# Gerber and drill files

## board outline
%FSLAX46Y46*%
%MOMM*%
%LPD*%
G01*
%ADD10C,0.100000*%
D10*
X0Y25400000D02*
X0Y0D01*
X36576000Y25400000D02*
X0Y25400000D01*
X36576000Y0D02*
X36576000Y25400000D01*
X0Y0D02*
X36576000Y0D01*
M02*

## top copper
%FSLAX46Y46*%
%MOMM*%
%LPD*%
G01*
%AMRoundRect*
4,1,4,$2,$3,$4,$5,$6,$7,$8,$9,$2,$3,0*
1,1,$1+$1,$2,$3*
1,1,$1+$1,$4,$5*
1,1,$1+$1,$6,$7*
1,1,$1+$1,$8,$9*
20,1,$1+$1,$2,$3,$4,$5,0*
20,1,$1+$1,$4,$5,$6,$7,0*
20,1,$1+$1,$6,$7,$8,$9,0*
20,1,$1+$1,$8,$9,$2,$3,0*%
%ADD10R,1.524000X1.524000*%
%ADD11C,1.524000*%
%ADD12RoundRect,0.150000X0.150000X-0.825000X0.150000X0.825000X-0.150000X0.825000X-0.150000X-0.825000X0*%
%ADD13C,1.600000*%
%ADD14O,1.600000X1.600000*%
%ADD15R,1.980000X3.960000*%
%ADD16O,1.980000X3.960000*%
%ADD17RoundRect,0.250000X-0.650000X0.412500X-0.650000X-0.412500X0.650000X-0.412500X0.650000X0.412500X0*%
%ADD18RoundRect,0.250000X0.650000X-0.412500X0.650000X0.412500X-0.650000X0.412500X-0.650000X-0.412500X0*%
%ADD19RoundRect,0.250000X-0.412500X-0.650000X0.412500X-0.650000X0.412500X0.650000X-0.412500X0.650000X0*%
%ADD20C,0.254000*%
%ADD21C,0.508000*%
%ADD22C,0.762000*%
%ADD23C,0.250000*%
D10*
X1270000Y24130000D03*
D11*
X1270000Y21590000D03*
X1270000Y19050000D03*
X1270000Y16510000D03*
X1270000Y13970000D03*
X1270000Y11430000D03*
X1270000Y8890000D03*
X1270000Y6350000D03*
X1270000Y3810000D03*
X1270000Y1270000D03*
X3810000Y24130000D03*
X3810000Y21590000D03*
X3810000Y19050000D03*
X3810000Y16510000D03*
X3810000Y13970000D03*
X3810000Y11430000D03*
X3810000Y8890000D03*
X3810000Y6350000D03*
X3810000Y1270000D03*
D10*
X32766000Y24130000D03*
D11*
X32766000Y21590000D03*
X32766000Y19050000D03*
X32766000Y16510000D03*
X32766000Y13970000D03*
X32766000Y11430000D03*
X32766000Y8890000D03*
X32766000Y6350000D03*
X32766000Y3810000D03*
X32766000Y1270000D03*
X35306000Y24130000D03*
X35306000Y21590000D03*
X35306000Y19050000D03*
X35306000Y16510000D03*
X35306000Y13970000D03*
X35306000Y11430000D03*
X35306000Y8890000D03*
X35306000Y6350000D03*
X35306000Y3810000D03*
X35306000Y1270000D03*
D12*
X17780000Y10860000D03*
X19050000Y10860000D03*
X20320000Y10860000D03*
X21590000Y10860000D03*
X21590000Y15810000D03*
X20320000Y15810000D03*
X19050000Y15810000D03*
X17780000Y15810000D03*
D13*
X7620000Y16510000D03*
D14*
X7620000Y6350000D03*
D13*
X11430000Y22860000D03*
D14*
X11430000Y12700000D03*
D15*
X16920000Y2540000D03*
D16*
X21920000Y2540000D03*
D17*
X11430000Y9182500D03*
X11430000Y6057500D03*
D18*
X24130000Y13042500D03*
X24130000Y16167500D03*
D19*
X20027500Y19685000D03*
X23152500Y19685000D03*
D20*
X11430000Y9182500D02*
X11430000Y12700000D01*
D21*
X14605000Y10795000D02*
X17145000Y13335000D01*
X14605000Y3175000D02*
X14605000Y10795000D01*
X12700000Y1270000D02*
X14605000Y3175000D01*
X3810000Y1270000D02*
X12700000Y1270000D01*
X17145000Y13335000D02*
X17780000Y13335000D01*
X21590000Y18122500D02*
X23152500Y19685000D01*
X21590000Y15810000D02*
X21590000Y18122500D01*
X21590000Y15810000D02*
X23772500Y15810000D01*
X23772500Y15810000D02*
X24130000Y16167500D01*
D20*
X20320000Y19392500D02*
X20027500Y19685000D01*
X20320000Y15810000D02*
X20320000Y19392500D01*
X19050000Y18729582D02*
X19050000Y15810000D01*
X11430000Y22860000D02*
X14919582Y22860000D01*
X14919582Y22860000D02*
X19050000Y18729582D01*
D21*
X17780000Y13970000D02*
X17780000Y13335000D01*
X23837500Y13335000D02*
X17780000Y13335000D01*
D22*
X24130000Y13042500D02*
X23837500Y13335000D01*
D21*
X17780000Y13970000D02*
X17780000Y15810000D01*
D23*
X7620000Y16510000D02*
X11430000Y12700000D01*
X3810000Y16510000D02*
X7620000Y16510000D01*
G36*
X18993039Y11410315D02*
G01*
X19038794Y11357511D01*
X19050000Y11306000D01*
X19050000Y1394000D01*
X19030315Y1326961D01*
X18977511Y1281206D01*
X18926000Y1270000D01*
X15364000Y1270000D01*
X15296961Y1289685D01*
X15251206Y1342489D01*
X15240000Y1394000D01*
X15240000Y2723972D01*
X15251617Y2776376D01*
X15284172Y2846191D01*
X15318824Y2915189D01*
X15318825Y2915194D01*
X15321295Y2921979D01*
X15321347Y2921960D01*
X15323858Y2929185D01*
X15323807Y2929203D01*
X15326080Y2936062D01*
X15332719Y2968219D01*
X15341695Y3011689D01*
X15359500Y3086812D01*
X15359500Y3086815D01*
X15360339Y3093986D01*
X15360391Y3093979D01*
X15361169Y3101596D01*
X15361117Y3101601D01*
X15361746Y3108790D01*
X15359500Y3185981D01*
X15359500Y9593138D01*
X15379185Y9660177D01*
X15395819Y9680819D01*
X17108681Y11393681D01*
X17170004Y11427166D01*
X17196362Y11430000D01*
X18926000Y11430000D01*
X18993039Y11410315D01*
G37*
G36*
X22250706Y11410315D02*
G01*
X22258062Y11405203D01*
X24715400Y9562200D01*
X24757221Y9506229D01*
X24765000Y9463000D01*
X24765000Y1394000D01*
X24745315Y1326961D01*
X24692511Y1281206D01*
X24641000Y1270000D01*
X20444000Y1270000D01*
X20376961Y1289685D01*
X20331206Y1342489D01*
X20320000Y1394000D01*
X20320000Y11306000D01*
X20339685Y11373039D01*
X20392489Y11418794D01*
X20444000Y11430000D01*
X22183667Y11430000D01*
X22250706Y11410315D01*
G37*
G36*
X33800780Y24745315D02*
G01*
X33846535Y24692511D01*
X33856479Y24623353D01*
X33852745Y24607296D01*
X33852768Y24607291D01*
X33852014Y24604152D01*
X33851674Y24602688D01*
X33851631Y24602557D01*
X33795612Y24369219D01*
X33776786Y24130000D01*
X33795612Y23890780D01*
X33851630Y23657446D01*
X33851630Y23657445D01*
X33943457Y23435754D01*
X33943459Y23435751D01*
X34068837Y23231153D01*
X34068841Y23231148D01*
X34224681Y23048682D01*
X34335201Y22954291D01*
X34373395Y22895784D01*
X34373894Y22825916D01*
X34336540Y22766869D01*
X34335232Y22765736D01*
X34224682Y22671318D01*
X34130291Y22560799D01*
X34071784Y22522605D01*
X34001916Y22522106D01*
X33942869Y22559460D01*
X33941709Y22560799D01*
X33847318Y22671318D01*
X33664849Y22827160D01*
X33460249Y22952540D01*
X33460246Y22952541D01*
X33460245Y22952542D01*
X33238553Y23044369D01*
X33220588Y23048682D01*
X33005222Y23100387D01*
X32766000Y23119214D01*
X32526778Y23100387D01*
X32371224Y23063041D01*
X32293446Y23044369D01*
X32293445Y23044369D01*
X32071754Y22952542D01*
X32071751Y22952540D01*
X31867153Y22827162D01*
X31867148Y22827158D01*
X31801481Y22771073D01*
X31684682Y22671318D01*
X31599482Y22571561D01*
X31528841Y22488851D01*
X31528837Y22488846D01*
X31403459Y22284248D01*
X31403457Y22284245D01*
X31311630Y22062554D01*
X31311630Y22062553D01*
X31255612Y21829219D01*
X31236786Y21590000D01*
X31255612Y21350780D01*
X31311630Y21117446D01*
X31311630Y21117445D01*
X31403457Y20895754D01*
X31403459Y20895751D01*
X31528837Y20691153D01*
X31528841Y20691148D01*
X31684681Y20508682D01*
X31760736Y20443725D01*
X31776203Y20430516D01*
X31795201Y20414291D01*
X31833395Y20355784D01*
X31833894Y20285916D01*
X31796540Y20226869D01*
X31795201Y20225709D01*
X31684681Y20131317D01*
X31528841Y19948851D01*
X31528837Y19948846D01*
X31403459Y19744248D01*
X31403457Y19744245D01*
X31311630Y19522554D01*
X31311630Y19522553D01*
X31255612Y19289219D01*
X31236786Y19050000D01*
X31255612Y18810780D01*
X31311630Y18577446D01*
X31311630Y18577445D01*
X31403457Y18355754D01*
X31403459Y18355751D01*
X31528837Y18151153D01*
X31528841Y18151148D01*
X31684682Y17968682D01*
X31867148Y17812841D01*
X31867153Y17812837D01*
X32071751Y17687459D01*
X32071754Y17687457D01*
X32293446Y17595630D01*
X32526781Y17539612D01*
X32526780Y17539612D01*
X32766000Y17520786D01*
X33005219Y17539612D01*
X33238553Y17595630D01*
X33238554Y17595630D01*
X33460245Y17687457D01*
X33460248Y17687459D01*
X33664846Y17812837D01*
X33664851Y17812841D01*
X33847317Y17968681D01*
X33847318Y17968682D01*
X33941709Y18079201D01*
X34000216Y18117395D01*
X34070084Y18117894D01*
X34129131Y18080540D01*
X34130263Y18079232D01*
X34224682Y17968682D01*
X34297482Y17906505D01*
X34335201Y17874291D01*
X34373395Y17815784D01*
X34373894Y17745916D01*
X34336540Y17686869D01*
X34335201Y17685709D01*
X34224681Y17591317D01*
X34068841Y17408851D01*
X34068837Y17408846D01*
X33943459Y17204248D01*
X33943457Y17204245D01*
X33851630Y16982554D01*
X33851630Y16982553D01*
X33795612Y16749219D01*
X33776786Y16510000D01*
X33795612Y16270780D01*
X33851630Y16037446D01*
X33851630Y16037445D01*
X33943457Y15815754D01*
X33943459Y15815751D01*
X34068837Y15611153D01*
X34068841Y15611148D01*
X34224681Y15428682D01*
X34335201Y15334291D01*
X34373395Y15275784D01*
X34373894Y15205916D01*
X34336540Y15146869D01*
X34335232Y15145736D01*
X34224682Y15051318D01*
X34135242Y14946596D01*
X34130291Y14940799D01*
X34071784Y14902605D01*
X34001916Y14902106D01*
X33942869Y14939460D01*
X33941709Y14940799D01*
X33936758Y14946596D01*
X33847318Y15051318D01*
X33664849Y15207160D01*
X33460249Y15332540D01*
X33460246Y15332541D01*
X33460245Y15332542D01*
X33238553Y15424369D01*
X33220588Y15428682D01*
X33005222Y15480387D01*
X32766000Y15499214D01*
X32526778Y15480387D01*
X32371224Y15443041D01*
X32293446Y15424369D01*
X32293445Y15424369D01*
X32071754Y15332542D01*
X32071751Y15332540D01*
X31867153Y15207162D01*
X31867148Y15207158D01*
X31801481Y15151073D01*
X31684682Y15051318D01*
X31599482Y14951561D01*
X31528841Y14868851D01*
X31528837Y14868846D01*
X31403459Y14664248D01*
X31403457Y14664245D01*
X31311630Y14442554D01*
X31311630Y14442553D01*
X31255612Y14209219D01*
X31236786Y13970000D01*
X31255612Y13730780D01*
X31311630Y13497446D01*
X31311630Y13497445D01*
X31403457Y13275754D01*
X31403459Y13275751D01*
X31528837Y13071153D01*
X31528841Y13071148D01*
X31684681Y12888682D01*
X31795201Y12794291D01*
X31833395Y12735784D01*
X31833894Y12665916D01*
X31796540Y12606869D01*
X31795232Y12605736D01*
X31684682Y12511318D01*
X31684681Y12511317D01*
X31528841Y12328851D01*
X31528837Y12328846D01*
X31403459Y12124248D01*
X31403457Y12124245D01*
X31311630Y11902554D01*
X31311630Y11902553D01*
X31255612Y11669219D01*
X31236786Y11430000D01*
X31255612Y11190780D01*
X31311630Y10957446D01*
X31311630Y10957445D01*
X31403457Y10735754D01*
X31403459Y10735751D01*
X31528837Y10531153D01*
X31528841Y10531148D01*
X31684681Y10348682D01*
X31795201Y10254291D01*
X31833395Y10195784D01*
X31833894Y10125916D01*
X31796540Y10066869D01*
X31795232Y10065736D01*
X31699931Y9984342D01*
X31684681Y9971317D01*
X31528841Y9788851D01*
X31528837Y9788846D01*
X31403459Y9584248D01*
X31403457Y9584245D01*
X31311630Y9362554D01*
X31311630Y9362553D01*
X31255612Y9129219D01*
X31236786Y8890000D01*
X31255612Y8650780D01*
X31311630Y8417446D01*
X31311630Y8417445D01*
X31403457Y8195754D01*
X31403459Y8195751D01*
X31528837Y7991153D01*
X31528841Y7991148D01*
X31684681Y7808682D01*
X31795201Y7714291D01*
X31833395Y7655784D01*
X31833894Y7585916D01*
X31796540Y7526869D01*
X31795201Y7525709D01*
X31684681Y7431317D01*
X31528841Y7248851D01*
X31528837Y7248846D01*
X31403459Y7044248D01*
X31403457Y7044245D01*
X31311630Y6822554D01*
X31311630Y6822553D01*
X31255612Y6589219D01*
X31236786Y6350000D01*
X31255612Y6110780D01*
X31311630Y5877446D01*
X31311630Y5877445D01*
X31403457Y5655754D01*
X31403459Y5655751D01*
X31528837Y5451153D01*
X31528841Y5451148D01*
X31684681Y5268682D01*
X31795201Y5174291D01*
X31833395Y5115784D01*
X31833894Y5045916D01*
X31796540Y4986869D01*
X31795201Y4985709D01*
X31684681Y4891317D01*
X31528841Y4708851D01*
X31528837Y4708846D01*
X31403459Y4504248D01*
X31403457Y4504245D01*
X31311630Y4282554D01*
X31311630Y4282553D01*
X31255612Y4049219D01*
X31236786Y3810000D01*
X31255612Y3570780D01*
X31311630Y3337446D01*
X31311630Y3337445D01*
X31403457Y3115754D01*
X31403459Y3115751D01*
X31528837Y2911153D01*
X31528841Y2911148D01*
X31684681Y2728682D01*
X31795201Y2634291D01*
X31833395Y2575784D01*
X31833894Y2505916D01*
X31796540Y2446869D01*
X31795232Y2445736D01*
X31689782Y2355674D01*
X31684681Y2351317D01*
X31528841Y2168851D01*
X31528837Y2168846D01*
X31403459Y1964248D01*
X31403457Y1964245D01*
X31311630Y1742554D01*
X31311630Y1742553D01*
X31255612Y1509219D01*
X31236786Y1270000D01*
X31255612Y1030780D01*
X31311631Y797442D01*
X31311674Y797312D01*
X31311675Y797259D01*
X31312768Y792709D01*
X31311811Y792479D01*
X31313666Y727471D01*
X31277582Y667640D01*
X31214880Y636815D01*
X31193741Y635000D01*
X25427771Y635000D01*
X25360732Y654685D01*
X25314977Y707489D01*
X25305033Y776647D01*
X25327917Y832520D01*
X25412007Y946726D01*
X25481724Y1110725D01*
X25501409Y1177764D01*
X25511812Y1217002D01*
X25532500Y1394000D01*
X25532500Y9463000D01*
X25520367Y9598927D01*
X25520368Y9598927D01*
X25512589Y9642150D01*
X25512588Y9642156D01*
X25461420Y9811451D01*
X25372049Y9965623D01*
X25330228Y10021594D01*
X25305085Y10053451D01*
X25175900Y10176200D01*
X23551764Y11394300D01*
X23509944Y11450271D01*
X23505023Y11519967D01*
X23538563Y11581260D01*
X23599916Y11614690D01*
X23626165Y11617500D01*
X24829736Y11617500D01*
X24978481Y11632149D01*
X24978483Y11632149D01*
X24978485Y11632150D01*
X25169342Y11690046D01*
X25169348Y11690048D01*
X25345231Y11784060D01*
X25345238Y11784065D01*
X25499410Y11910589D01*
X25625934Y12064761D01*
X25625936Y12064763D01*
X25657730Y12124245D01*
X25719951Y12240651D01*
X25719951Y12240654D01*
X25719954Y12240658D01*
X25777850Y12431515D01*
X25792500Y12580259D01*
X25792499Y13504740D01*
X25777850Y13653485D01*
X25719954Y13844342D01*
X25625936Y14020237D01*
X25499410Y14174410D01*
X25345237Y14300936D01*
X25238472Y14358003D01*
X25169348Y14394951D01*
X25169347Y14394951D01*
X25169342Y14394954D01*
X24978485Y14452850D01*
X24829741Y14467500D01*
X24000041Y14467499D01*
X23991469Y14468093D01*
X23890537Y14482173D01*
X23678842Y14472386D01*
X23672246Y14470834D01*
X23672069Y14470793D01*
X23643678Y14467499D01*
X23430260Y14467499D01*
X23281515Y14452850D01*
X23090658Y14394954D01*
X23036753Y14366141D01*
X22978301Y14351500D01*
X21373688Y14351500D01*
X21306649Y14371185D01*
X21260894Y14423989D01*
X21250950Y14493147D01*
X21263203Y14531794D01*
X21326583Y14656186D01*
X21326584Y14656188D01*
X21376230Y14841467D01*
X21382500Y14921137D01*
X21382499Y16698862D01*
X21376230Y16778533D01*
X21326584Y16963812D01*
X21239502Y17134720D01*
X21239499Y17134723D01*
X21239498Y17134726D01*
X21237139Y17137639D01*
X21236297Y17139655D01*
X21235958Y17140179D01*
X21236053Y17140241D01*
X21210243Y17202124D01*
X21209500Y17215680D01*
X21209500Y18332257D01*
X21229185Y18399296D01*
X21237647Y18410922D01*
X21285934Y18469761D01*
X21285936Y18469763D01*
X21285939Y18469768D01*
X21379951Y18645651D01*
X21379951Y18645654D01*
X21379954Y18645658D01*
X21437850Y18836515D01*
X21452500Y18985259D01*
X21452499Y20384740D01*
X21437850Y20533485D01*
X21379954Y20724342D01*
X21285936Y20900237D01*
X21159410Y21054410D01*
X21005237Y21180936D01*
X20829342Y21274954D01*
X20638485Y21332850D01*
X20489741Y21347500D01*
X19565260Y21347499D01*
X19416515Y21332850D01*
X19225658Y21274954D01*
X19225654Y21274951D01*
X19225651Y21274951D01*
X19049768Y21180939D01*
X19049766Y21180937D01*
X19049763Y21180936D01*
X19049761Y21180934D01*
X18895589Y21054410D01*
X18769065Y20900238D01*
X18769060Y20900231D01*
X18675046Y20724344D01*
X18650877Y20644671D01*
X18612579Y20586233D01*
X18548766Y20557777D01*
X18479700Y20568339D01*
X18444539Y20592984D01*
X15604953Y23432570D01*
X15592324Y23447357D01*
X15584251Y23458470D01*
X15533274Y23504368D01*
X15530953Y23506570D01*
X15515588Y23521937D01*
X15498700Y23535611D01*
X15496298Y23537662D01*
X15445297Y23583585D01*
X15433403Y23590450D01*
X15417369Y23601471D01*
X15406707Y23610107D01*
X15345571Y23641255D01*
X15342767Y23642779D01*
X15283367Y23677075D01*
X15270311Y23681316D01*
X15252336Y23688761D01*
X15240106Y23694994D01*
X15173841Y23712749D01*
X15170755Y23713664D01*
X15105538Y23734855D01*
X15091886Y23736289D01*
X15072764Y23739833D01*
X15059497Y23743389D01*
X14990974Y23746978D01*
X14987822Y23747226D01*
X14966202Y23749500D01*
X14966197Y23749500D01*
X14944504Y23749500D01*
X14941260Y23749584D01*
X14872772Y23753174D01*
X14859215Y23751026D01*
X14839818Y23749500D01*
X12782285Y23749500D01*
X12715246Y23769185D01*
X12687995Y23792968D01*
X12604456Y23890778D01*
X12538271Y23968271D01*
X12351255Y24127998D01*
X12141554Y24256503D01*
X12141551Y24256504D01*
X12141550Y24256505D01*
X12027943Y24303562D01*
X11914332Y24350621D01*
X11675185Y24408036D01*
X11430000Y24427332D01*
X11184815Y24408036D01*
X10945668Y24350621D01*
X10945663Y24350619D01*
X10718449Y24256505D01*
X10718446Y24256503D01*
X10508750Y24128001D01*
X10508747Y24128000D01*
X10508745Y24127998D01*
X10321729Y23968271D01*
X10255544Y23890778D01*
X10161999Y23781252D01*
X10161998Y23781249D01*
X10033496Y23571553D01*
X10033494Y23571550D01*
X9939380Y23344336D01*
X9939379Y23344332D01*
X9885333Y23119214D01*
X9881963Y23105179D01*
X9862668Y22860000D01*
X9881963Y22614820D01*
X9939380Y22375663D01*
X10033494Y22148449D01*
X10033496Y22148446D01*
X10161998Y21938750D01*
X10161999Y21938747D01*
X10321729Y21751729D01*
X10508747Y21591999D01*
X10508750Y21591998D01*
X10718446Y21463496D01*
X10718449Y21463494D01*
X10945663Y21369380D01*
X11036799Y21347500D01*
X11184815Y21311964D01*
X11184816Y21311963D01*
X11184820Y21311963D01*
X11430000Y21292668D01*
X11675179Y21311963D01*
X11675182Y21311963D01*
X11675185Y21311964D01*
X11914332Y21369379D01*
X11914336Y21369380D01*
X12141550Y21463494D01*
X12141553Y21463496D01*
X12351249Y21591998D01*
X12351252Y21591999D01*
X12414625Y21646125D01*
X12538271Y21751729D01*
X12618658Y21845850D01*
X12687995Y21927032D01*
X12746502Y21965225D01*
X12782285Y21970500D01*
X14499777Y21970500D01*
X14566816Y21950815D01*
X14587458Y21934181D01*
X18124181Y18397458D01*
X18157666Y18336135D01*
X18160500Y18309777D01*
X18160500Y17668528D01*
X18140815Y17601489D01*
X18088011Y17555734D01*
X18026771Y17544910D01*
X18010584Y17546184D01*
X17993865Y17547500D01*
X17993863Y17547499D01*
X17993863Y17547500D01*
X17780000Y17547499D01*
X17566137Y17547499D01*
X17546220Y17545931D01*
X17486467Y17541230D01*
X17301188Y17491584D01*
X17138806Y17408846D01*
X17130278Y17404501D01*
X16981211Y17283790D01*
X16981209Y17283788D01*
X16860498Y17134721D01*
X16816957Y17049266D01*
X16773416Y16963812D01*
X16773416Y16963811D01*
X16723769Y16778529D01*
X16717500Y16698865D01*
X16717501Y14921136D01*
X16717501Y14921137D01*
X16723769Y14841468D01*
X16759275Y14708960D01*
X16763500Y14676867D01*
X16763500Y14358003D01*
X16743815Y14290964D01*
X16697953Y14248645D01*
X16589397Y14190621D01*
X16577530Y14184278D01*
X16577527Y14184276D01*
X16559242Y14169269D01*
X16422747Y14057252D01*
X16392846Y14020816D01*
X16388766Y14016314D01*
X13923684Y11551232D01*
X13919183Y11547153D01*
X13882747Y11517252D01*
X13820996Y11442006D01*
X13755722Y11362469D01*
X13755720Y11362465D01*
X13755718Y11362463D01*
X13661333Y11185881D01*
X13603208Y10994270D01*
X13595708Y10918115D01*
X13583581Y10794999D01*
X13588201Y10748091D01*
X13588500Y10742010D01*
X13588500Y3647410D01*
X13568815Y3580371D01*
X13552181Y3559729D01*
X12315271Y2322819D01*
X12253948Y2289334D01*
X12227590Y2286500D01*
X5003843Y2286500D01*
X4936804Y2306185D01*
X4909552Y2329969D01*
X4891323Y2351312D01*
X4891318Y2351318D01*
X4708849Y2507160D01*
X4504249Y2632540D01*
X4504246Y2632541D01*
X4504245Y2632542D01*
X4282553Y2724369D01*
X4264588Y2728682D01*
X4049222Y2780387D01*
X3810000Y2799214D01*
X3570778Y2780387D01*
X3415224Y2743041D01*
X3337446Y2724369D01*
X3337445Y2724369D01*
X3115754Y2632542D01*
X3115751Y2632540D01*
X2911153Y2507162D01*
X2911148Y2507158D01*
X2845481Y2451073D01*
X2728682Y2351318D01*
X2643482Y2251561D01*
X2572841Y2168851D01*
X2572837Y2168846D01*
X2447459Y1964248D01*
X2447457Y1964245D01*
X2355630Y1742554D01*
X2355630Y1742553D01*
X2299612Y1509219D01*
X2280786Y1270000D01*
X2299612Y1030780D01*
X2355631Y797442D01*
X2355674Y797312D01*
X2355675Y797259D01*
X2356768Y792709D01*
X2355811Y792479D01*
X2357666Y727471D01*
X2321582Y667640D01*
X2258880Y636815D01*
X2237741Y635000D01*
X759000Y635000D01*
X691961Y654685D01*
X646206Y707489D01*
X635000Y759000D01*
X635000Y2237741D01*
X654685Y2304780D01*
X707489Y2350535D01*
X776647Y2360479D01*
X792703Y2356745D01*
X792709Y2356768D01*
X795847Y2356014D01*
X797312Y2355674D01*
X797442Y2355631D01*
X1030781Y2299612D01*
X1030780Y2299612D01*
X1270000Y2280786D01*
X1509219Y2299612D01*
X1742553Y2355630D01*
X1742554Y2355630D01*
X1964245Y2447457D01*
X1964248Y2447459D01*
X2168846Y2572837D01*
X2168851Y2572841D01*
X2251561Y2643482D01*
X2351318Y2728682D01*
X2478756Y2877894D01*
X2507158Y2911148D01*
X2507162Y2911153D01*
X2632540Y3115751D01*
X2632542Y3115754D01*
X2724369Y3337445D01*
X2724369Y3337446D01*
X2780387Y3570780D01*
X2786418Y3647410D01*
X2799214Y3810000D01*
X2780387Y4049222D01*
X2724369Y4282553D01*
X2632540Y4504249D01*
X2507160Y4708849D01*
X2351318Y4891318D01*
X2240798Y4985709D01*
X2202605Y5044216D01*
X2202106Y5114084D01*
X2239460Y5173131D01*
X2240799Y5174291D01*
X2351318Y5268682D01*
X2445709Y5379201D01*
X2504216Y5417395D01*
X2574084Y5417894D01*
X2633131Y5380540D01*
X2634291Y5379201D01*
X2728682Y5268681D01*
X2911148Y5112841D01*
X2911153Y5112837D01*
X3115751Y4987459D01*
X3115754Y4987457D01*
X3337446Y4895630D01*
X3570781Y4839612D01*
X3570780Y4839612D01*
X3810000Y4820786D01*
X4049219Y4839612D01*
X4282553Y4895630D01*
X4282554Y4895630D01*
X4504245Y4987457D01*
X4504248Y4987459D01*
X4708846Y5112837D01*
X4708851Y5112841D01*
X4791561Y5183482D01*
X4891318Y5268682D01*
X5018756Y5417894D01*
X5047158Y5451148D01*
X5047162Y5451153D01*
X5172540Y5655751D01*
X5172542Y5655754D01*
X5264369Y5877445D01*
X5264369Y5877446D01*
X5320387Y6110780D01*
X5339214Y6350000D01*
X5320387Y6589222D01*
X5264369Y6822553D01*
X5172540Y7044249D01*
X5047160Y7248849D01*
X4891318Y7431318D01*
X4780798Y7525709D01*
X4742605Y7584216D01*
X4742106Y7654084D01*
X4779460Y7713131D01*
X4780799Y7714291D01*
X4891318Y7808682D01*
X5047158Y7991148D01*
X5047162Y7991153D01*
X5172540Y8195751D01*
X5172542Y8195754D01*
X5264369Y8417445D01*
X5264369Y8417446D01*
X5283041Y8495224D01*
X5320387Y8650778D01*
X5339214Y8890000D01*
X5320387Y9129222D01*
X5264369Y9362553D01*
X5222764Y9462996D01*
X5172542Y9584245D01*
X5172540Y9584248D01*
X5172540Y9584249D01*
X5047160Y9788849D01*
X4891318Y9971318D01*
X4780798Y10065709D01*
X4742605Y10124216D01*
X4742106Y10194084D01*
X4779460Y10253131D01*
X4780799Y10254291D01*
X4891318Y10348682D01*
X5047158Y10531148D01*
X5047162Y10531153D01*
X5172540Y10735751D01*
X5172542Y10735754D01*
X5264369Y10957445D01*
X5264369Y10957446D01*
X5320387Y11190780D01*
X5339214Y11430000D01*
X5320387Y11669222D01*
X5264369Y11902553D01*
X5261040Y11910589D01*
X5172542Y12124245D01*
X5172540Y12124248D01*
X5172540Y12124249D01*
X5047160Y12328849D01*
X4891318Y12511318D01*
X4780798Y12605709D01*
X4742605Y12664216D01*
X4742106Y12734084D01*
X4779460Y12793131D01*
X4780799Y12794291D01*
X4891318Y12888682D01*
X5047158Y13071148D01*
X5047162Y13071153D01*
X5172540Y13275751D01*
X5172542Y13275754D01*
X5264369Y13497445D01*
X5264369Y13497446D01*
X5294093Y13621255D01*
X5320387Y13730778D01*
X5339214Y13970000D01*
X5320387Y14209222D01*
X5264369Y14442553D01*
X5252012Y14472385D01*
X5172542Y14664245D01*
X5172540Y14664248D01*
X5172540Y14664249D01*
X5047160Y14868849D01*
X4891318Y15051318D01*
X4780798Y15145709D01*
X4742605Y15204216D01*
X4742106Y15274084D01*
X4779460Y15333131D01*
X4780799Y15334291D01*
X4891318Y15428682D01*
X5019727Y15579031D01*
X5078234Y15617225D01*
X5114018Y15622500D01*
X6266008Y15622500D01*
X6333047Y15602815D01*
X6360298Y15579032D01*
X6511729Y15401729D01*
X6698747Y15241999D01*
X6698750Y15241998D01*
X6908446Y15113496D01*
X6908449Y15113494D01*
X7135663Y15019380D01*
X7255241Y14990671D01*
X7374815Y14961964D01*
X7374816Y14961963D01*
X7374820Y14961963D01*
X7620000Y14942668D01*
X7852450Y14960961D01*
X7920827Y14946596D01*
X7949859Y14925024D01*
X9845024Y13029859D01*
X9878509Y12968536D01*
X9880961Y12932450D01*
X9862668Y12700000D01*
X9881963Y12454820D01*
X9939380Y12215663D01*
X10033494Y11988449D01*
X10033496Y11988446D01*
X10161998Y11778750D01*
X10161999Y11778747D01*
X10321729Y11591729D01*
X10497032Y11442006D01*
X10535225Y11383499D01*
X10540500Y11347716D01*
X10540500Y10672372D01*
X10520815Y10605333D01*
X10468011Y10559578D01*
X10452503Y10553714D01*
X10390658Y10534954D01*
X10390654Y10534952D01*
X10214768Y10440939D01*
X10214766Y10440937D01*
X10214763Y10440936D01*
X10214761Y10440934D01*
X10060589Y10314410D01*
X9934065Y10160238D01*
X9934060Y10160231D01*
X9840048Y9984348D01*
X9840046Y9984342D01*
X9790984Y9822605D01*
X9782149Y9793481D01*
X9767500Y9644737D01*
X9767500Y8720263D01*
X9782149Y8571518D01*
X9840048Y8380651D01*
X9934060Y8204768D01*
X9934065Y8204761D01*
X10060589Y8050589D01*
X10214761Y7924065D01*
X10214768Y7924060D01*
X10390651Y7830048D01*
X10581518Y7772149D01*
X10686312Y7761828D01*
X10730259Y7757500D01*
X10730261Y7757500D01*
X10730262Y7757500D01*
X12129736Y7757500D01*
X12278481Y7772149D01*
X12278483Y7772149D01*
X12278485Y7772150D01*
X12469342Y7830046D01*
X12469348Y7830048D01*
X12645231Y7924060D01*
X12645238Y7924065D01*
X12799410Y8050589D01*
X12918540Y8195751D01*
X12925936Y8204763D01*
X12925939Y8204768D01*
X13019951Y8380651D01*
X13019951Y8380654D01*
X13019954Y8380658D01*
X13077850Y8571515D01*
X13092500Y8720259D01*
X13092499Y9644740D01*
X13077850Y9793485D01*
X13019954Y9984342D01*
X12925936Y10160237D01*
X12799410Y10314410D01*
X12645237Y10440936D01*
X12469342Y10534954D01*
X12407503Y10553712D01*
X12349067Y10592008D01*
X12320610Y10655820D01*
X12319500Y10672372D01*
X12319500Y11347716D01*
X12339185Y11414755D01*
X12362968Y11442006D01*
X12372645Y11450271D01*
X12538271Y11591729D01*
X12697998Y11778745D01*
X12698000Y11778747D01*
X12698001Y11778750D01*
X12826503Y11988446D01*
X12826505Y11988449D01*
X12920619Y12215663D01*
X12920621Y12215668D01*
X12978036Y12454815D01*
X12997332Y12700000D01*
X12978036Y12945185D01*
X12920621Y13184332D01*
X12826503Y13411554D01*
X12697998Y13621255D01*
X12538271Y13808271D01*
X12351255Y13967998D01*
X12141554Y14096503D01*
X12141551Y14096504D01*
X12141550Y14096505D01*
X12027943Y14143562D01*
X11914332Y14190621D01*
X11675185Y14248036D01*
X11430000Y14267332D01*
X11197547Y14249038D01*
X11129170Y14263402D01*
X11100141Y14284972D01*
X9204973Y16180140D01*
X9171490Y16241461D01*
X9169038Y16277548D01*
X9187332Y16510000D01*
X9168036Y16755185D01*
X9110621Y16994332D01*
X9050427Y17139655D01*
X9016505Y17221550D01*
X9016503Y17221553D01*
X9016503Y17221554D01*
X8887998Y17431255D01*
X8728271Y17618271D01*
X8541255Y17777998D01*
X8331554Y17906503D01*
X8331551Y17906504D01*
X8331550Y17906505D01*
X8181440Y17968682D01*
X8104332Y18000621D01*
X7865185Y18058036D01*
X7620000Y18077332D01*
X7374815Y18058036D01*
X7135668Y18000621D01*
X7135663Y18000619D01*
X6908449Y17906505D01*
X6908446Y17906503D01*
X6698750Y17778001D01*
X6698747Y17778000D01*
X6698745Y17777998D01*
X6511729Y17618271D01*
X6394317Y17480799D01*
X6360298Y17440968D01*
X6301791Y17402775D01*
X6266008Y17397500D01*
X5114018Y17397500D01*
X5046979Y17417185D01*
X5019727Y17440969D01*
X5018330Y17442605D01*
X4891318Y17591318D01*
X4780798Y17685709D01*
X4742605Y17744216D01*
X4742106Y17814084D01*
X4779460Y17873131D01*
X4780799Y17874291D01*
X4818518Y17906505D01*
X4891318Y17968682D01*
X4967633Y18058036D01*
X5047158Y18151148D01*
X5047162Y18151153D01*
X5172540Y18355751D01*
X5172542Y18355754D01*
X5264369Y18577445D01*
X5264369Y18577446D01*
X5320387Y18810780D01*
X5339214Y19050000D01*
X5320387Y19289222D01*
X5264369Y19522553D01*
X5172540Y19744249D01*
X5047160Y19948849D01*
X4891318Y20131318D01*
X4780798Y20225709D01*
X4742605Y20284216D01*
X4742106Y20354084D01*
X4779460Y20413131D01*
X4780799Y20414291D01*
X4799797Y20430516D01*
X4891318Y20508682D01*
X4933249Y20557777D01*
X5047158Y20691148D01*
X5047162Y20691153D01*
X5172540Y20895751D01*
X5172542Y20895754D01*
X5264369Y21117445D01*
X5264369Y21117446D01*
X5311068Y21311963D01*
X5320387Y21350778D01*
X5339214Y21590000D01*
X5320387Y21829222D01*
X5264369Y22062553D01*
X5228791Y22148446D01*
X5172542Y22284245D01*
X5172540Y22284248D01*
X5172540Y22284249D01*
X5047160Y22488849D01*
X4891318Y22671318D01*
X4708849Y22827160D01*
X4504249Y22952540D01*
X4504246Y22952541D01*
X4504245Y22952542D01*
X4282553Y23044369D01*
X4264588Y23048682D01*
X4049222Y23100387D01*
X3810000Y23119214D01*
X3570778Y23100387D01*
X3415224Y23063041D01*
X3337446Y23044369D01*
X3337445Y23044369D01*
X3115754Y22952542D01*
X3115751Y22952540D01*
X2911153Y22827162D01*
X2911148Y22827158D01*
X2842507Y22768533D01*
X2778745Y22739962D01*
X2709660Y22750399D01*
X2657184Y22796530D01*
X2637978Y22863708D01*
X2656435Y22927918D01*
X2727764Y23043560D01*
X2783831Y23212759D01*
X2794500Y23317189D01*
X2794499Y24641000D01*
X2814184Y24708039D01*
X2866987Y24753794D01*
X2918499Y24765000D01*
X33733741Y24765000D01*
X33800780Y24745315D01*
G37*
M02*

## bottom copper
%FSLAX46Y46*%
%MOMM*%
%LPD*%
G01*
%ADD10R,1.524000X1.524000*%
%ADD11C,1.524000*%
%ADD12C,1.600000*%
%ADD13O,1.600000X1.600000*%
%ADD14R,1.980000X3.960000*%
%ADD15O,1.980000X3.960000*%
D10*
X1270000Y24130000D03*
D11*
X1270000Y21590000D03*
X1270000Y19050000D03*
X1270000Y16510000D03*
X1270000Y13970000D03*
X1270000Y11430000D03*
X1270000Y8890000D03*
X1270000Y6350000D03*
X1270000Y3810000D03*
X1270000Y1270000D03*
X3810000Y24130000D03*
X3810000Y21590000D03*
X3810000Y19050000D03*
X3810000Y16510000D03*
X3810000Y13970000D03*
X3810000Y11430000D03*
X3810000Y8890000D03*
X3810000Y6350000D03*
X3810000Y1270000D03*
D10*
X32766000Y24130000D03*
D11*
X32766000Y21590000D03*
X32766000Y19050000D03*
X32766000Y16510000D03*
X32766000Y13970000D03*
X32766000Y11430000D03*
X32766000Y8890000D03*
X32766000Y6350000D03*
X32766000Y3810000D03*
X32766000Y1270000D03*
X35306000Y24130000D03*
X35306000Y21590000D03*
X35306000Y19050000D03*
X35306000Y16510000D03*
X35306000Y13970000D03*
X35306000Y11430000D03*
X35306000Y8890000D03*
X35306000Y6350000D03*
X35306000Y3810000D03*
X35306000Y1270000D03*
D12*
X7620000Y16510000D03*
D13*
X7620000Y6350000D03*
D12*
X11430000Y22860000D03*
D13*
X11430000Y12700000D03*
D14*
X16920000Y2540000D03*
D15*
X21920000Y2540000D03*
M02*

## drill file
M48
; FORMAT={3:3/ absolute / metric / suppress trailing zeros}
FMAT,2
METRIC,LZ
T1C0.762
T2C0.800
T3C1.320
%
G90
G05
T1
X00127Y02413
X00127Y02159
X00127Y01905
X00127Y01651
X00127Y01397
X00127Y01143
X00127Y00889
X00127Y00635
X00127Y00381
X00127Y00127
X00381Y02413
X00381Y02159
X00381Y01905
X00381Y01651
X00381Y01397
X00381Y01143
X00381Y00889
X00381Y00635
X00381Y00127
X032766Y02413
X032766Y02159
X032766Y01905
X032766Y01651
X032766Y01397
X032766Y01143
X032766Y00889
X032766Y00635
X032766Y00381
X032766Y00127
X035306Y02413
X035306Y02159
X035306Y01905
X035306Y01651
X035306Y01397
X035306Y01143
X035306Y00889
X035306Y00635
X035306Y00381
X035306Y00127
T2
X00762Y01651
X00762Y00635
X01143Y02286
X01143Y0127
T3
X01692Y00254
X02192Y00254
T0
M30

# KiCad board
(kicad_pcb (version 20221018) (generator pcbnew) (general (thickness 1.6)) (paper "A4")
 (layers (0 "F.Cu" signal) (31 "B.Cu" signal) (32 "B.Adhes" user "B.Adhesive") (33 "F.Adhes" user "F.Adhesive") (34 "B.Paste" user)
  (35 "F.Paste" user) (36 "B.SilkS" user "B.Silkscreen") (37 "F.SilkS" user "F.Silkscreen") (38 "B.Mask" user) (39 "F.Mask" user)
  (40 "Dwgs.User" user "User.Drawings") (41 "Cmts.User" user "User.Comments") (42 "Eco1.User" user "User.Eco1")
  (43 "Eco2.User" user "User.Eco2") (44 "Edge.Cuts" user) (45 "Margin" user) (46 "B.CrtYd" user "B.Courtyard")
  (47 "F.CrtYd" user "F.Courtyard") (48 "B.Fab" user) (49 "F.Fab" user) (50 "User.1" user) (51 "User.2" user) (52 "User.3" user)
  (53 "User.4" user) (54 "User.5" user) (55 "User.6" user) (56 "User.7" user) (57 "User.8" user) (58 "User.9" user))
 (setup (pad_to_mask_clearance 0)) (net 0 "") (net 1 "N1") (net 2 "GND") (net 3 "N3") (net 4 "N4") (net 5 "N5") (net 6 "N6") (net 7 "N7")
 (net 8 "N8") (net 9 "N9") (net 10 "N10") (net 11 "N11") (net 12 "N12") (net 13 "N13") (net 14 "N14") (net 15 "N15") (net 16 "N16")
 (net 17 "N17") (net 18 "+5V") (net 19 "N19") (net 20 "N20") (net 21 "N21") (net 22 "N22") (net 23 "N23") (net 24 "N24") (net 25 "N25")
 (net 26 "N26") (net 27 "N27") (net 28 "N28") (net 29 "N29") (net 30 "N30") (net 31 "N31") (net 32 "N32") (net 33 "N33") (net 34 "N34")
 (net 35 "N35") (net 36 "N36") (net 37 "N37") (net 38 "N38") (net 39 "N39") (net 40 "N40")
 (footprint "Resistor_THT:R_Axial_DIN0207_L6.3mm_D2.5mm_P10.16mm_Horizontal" (layer "F.Cu") (at 7.62 -16.51 -90)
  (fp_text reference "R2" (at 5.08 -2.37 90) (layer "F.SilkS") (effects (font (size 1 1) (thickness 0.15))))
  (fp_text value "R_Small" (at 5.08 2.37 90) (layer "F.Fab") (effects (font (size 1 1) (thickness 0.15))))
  (pad "1" thru_hole circle (at 0 0 270) (size 1.6 1.6) (drill 0.8) (layers "*.Cu" "*.Mask") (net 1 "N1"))
  (pad "2" thru_hole oval (at 10.16 0 270) (size 1.6 1.6) (drill 0.8) (layers "*.Cu" "*.Mask") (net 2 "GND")))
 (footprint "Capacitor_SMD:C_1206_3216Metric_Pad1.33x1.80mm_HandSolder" (layer "F.Cu") (at 11.43 -7.62 -90)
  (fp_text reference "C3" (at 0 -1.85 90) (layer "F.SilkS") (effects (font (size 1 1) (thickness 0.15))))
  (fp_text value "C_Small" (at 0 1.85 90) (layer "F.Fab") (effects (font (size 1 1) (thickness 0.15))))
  (pad "1" smd roundrect (at -1.5625 0 270) (size 1.325 1.8) (layers "F.Cu" "F.Paste" "F.Mask") (roundrect_rratio 0.1886792453) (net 1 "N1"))
  (pad "2" smd roundrect (at 1.5625 0 270) (size 1.325 1.8) (layers "F.Cu" "F.Paste" "F.Mask") (roundrect_rratio 0.1886792453) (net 2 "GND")))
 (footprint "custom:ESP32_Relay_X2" (layer "F.Cu") (at 35.306 -13.97)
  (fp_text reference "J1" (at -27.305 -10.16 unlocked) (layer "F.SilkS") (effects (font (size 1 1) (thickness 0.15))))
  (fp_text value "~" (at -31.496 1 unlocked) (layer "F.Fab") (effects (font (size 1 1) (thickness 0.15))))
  (pad "1" thru_hole rect (at -34.036 -10.16) (size 1.524 1.524) (drill 0.762) (layers "*.Cu" "*.Mask") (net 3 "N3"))
  (pad "2" thru_hole circle (at -34.036 -7.62) (size 1.524 1.524) (drill 0.762) (layers "*.Cu" "*.Mask") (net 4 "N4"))
  (pad "3" thru_hole circle (at -34.036 -5.08) (size 1.524 1.524) (drill 0.762) (layers "*.Cu" "*.Mask") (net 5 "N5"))
  (pad "4" thru_hole circle (at -34.036 -2.54) (size 1.524 1.524) (drill 0.762) (layers "*.Cu" "*.Mask") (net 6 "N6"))
  (pad "5" thru_hole circle (at -34.036 0) (size 1.524 1.524) (drill 0.762) (layers "*.Cu" "*.Mask") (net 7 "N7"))
  (pad "6" thru_hole circle (at -34.036 2.54) (size 1.524 1.524) (drill 0.762) (layers "*.Cu" "*.Mask") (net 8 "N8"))
  (pad "7" thru_hole circle (at -34.036 5.08) (size 1.524 1.524) (drill 0.762) (layers "*.Cu" "*.Mask") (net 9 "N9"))
  (pad "8" thru_hole circle (at -34.036 7.62) (size 1.524 1.524) (drill 0.762) (layers "*.Cu" "*.Mask") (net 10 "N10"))
  (pad "9" thru_hole circle (at -34.036 10.16) (size 1.524 1.524) (drill 0.762) (layers "*.Cu" "*.Mask") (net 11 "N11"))
  (pad "10" thru_hole circle (at -34.036 12.7) (size 1.524 1.524) (drill 0.762) (layers "*.Cu" "*.Mask") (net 2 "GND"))
  (pad "11" thru_hole circle (at -31.496 -10.16) (size 1.524 1.524) (drill 0.762) (layers "*.Cu" "*.Mask") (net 2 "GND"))
  (pad "12" thru_hole circle (at -31.496 -7.62) (size 1.524 1.524) (drill 0.762) (layers "*.Cu" "*.Mask") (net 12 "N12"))
  (pad "13" thru_hole circle (at -31.496 -5.08) (size 1.524 1.524) (drill 0.762) (layers "*.Cu" "*.Mask") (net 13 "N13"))
  (pad "14" thru_hole circle (at -31.496 -2.54) (size 1.524 1.524) (drill 0.762) (layers "*.Cu" "*.Mask") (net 1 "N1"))
  (pad "15" thru_hole circle (at -31.496 0) (size 1.524 1.524) (drill 0.762) (layers "*.Cu" "*.Mask") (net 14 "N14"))
  (pad "16" thru_hole circle (at -31.496 2.54) (size 1.524 1.524) (drill 0.762) (layers "*.Cu" "*.Mask") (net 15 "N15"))
  (pad "17" thru_hole circle (at -31.496 5.08) (size 1.524 1.524) (drill 0.762) (layers "*.Cu" "*.Mask") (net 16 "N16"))
  (pad "18" thru_hole circle (at -31.496 7.62) (size 1.524 1.524) (drill 0.762) (layers "*.Cu" "*.Mask") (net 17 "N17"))
  (pad "20" thru_hole circle (at -31.496 12.7) (size 1.524 1.524) (drill 0.762) (layers "*.Cu" "*.Mask") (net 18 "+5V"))
  (pad "21" thru_hole rect (at -2.54 -10.16) (size 1.524 1.524) (drill 0.762) (layers "*.Cu" "*.Mask") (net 2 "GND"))
  (pad "22" thru_hole circle (at -2.54 -7.62) (size 1.524 1.524) (drill 0.762) (layers "*.Cu" "*.Mask") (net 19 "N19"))
  (pad "23" thru_hole circle (at -2.54 -5.08) (size 1.524 1.524) (drill 0.762) (layers "*.Cu" "*.Mask") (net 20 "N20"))
  (pad "24" thru_hole circle (at -2.54 -2.54) (size 1.524 1.524) (drill 0.762) (layers "*.Cu" "*.Mask") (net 2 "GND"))
  (pad "25" thru_hole circle (at -2.54 0) (size 1.524 1.524) (drill 0.762) (layers "*.Cu" "*.Mask") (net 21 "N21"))
  (pad "26" thru_hole circle (at -2.54 2.54) (size 1.524 1.524) (drill 0.762) (layers "*.Cu" "*.Mask") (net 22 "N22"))
  (pad "27" thru_hole circle (at -2.54 5.08) (size 1.524 1.524) (drill 0.762) (layers "*.Cu" "*.Mask") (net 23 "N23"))
  (pad "28" thru_hole circle (at -2.54 7.62) (size 1.524 1.524) (drill 0.762) (layers "*.Cu" "*.Mask") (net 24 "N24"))
  (pad "29" thru_hole circle (at -2.54 10.16) (size 1.524 1.524) (drill 0.762) (layers "*.Cu" "*.Mask") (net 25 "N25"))
  (pad "30" thru_hole circle (at -2.54 12.7) (size 1.524 1.524) (drill 0.762) (layers "*.Cu" "*.Mask") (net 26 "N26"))
  (pad "31" thru_hole circle (at 0 -10.16) (size 1.524 1.524) (drill 0.762) (layers "*.Cu" "*.Mask") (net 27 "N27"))
  (pad "32" thru_hole circle (at 0 -7.62) (size 1.524 1.524) (drill 0.762) (layers "*.Cu" "*.Mask") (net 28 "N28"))
  (pad "33" thru_hole circle (at 0 -5.08) (size 1.524 1.524) (drill 0.762) (layers "*.Cu" "*.Mask") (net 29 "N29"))
  (pad "34" thru_hole circle (at 0 -2.54) (size 1.524 1.524) (drill 0.762) (layers "*.Cu" "*.Mask") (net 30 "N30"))
  (pad "35" thru_hole circle (at 0 0) (size 1.524 1.524) (drill 0.762) (layers "*.Cu" "*.Mask") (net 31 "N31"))
  (pad "36" thru_hole circle (at 0 2.54) (size 1.524 1.524) (drill 0.762) (layers "*.Cu" "*.Mask") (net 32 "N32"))
  (pad "37" thru_hole circle (at 0 5.08) (size 1.524 1.524) (drill 0.762) (layers "*.Cu" "*.Mask") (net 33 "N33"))
  (pad "38" thru_hole circle (at 0 7.62) (size 1.524 1.524) (drill 0.762) (layers "*.Cu" "*.Mask") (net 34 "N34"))
  (pad "39" thru_hole circle (at 0 10.16) (size 1.524 1.524) (drill 0.762) (layers "*.Cu" "*.Mask") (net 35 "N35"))
  (pad "40" thru_hole circle (at 0 12.7) (size 1.524 1.524) (drill 0.762) (layers "*.Cu" "*.Mask") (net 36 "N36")))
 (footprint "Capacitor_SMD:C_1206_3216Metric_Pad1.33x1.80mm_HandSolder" (layer "F.Cu") (at 21.59 -19.685)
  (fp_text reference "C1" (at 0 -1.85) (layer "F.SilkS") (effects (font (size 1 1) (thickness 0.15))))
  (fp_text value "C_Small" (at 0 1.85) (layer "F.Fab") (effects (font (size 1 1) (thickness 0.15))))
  (pad "1" smd roundrect (at -1.5625 0) (size 1.325 1.8) (layers "F.Cu" "F.Paste" "F.Mask") (roundrect_rratio 0.1886792453) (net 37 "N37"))
  (pad "2" smd roundrect (at 1.5625 0) (size 1.325 1.8) (layers "F.Cu" "F.Paste" "F.Mask") (roundrect_rratio 0.1886792453) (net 2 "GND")))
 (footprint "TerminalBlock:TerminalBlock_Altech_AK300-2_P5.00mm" (layer "F.Cu") (at 16.92 -2.54)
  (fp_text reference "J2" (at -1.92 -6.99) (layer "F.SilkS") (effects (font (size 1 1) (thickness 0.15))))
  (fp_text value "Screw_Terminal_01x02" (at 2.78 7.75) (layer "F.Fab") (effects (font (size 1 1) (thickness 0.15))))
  (pad "1" thru_hole rect (at 0 0) (size 1.98 3.96) (drill 1.32) (layers "*.Cu" "*.Mask") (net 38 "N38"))
  (pad "2" thru_hole oval (at 5 0) (size 1.98 3.96) (drill 1.32) (layers "*.Cu" "*.Mask") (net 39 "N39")))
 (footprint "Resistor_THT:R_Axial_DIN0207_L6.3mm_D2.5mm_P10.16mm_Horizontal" (layer "F.Cu") (at 11.43 -22.86 -90)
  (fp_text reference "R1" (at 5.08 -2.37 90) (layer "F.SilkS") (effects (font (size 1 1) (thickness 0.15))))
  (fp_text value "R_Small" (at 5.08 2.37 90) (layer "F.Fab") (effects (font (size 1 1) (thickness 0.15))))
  (pad "1" thru_hole circle (at 0 0 270) (size 1.6 1.6) (drill 0.8) (layers "*.Cu" "*.Mask") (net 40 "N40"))
  (pad "2" thru_hole oval (at 10.16 0 270) (size 1.6 1.6) (drill 0.8) (layers "*.Cu" "*.Mask") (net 1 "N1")))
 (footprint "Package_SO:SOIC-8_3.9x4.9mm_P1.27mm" (layer "F.Cu") (at 19.685 -13.335 90)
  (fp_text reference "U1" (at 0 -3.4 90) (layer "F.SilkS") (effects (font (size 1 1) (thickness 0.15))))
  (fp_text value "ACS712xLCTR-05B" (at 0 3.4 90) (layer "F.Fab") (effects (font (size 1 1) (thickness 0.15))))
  (pad "1" smd roundrect (at -2.475 -1.905 90) (size 1.95 0.6) (layers "F.Cu" "F.Paste" "F.Mask") (roundrect_rratio 0.25) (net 38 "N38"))
  (pad "2" smd roundrect (at -2.475 -0.635 90) (size 1.95 0.6) (layers "F.Cu" "F.Paste" "F.Mask") (roundrect_rratio 0.25) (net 38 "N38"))
  (pad "3" smd roundrect (at -2.475 0.635 90) (size 1.95 0.6) (layers "F.Cu" "F.Paste" "F.Mask") (roundrect_rratio 0.25) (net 39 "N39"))
  (pad "4" smd roundrect (at -2.475 1.905 90) (size 1.95 0.6) (layers "F.Cu" "F.Paste" "F.Mask") (roundrect_rratio 0.25) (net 39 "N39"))
  (pad "5" smd roundrect (at 2.475 1.905 90) (size 1.95 0.6) (layers "F.Cu" "F.Paste" "F.Mask") (roundrect_rratio 0.25) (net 2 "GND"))
  (pad "6" smd roundrect (at 2.475 0.635 90) (size 1.95 0.6) (layers "F.Cu" "F.Paste" "F.Mask") (roundrect_rratio 0.25) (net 37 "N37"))
  (pad "7" smd roundrect (at 2.475 -0.635 90) (size 1.95 0.6) (layers "F.Cu" "F.Paste" "F.Mask") (roundrect_rratio 0.25) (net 40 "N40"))
  (pad "8" smd roundrect (at 2.475 -1.905 90) (size 1.95 0.6) (layers "F.Cu" "F.Paste" "F.Mask") (roundrect_rratio 0.25) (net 18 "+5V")))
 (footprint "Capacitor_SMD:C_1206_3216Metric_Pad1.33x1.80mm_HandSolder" (layer "F.Cu") (at 24.13 -14.605 90)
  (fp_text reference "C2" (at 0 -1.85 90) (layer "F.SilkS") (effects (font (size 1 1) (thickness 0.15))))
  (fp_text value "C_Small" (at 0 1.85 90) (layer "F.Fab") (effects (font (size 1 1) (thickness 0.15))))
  (pad "1" smd roundrect (at -1.5625 0 90) (size 1.325 1.8) (layers "F.Cu" "F.Paste" "F.Mask") (roundrect_rratio 0.1886792453)
   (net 18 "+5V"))
  (pad "2" smd roundrect (at 1.5625 0 90) (size 1.325 1.8) (layers "F.Cu" "F.Paste" "F.Mask") (roundrect_rratio 0.1886792453) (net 2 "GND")))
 (gr_line (start 0 0) (end 36.576 0) (stroke (width 0.1) (type default)) (layer "Edge.Cuts"))
 (gr_line (start 36.576 -25.4) (end 0 -25.4) (stroke (width 0.1) (type default)) (layer "Edge.Cuts"))
 (gr_line (start 36.576 0) (end 36.576 -25.4) (stroke (width 0.1) (type default)) (layer "Edge.Cuts"))
 (gr_line (start 0 -25.4) (end 0 0) (stroke (width 0.1) (type default)) (layer "Edge.Cuts"))
 (segment (start 20.32 -19.3925) (end 20.0275 -19.685) (width 0.254) (layer "F.Cu") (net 37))
 (segment (start 20.32 -15.81) (end 20.32 -19.3925) (width 0.254) (layer "F.Cu") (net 37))
 (segment (start 21.59 -18.1225) (end 23.1525 -19.685) (width 0.508) (layer "F.Cu") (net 2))
 (segment (start 21.59 -15.81) (end 23.7725 -15.81) (width 0.508) (layer "F.Cu") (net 2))
 (segment (start 21.59 -15.81) (end 21.59 -18.1225) (width 0.508) (layer "F.Cu") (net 2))
 (segment (start 23.7725 -15.81) (end 24.13 -16.1675) (width 0.508) (layer "F.Cu") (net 2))
 (segment (start 12.7 -1.27) (end 14.605 -3.175) (width 0.508) (layer "F.Cu") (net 18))
 (segment (start 14.605 -3.175) (end 14.605 -10.795) (width 0.508) (layer "F.Cu") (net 18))
 (segment (start 14.605 -10.795) (end 17.145 -13.335) (width 0.508) (layer "F.Cu") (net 18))
 (segment (start 24.13 -13.0425) (end 23.8375 -13.335) (width 0.762) (layer "F.Cu") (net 18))
 (segment (start 23.8375 -13.335) (end 17.78 -13.335) (width 0.508) (layer "F.Cu") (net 18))
 (segment (start 17.78 -13.97) (end 17.78 -15.81) (width 0.508) (layer "F.Cu") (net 18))
 (segment (start 17.78 -13.97) (end 17.78 -13.335) (width 0.508) (layer "F.Cu") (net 18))
 (segment (start 3.81 -1.27) (end 12.7 -1.27) (width 0.508) (layer "F.Cu") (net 18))
 (segment (start 17.145 -13.335) (end 17.78 -13.335) (width 0.508) (layer "F.Cu") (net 18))
 (segment (start 7.62 -16.51) (end 11.43 -12.7) (width 0.25) (layer "F.Cu") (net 1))
 (segment (start 11.43 -9.1825) (end 11.43 -12.7) (width 0.254) (layer "F.Cu") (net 1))
 (segment (start 3.81 -16.51) (end 7.62 -16.51) (width 0.25) (layer "F.Cu") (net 1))
 (segment (start 14.919582 -22.86) (end 19.05 -18.729582) (width 0.254) (layer "F.Cu") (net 40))
 (segment (start 11.43 -22.86) (end 14.919582 -22.86) (width 0.254) (layer "F.Cu") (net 40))
 (segment (start 19.05 -18.729582) (end 19.05 -15.81) (width 0.254) (layer "F.Cu") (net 40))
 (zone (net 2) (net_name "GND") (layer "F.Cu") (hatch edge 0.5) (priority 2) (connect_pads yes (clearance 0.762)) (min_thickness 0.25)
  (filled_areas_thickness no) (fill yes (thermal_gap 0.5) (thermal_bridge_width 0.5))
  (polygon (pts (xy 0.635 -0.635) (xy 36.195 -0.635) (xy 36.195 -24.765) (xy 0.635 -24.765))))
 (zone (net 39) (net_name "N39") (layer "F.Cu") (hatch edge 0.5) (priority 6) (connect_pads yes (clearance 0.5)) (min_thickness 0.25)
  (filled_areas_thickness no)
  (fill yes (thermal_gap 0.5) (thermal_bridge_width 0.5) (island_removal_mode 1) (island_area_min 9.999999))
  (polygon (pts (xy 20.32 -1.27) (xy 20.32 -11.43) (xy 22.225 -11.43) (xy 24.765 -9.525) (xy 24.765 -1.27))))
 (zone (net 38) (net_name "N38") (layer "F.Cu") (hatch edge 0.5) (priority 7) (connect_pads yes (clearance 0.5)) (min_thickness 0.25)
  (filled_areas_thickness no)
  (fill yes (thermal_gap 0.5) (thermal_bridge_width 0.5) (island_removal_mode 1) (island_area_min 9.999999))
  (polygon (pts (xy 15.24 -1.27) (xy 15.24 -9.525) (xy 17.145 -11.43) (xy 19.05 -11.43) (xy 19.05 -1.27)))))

